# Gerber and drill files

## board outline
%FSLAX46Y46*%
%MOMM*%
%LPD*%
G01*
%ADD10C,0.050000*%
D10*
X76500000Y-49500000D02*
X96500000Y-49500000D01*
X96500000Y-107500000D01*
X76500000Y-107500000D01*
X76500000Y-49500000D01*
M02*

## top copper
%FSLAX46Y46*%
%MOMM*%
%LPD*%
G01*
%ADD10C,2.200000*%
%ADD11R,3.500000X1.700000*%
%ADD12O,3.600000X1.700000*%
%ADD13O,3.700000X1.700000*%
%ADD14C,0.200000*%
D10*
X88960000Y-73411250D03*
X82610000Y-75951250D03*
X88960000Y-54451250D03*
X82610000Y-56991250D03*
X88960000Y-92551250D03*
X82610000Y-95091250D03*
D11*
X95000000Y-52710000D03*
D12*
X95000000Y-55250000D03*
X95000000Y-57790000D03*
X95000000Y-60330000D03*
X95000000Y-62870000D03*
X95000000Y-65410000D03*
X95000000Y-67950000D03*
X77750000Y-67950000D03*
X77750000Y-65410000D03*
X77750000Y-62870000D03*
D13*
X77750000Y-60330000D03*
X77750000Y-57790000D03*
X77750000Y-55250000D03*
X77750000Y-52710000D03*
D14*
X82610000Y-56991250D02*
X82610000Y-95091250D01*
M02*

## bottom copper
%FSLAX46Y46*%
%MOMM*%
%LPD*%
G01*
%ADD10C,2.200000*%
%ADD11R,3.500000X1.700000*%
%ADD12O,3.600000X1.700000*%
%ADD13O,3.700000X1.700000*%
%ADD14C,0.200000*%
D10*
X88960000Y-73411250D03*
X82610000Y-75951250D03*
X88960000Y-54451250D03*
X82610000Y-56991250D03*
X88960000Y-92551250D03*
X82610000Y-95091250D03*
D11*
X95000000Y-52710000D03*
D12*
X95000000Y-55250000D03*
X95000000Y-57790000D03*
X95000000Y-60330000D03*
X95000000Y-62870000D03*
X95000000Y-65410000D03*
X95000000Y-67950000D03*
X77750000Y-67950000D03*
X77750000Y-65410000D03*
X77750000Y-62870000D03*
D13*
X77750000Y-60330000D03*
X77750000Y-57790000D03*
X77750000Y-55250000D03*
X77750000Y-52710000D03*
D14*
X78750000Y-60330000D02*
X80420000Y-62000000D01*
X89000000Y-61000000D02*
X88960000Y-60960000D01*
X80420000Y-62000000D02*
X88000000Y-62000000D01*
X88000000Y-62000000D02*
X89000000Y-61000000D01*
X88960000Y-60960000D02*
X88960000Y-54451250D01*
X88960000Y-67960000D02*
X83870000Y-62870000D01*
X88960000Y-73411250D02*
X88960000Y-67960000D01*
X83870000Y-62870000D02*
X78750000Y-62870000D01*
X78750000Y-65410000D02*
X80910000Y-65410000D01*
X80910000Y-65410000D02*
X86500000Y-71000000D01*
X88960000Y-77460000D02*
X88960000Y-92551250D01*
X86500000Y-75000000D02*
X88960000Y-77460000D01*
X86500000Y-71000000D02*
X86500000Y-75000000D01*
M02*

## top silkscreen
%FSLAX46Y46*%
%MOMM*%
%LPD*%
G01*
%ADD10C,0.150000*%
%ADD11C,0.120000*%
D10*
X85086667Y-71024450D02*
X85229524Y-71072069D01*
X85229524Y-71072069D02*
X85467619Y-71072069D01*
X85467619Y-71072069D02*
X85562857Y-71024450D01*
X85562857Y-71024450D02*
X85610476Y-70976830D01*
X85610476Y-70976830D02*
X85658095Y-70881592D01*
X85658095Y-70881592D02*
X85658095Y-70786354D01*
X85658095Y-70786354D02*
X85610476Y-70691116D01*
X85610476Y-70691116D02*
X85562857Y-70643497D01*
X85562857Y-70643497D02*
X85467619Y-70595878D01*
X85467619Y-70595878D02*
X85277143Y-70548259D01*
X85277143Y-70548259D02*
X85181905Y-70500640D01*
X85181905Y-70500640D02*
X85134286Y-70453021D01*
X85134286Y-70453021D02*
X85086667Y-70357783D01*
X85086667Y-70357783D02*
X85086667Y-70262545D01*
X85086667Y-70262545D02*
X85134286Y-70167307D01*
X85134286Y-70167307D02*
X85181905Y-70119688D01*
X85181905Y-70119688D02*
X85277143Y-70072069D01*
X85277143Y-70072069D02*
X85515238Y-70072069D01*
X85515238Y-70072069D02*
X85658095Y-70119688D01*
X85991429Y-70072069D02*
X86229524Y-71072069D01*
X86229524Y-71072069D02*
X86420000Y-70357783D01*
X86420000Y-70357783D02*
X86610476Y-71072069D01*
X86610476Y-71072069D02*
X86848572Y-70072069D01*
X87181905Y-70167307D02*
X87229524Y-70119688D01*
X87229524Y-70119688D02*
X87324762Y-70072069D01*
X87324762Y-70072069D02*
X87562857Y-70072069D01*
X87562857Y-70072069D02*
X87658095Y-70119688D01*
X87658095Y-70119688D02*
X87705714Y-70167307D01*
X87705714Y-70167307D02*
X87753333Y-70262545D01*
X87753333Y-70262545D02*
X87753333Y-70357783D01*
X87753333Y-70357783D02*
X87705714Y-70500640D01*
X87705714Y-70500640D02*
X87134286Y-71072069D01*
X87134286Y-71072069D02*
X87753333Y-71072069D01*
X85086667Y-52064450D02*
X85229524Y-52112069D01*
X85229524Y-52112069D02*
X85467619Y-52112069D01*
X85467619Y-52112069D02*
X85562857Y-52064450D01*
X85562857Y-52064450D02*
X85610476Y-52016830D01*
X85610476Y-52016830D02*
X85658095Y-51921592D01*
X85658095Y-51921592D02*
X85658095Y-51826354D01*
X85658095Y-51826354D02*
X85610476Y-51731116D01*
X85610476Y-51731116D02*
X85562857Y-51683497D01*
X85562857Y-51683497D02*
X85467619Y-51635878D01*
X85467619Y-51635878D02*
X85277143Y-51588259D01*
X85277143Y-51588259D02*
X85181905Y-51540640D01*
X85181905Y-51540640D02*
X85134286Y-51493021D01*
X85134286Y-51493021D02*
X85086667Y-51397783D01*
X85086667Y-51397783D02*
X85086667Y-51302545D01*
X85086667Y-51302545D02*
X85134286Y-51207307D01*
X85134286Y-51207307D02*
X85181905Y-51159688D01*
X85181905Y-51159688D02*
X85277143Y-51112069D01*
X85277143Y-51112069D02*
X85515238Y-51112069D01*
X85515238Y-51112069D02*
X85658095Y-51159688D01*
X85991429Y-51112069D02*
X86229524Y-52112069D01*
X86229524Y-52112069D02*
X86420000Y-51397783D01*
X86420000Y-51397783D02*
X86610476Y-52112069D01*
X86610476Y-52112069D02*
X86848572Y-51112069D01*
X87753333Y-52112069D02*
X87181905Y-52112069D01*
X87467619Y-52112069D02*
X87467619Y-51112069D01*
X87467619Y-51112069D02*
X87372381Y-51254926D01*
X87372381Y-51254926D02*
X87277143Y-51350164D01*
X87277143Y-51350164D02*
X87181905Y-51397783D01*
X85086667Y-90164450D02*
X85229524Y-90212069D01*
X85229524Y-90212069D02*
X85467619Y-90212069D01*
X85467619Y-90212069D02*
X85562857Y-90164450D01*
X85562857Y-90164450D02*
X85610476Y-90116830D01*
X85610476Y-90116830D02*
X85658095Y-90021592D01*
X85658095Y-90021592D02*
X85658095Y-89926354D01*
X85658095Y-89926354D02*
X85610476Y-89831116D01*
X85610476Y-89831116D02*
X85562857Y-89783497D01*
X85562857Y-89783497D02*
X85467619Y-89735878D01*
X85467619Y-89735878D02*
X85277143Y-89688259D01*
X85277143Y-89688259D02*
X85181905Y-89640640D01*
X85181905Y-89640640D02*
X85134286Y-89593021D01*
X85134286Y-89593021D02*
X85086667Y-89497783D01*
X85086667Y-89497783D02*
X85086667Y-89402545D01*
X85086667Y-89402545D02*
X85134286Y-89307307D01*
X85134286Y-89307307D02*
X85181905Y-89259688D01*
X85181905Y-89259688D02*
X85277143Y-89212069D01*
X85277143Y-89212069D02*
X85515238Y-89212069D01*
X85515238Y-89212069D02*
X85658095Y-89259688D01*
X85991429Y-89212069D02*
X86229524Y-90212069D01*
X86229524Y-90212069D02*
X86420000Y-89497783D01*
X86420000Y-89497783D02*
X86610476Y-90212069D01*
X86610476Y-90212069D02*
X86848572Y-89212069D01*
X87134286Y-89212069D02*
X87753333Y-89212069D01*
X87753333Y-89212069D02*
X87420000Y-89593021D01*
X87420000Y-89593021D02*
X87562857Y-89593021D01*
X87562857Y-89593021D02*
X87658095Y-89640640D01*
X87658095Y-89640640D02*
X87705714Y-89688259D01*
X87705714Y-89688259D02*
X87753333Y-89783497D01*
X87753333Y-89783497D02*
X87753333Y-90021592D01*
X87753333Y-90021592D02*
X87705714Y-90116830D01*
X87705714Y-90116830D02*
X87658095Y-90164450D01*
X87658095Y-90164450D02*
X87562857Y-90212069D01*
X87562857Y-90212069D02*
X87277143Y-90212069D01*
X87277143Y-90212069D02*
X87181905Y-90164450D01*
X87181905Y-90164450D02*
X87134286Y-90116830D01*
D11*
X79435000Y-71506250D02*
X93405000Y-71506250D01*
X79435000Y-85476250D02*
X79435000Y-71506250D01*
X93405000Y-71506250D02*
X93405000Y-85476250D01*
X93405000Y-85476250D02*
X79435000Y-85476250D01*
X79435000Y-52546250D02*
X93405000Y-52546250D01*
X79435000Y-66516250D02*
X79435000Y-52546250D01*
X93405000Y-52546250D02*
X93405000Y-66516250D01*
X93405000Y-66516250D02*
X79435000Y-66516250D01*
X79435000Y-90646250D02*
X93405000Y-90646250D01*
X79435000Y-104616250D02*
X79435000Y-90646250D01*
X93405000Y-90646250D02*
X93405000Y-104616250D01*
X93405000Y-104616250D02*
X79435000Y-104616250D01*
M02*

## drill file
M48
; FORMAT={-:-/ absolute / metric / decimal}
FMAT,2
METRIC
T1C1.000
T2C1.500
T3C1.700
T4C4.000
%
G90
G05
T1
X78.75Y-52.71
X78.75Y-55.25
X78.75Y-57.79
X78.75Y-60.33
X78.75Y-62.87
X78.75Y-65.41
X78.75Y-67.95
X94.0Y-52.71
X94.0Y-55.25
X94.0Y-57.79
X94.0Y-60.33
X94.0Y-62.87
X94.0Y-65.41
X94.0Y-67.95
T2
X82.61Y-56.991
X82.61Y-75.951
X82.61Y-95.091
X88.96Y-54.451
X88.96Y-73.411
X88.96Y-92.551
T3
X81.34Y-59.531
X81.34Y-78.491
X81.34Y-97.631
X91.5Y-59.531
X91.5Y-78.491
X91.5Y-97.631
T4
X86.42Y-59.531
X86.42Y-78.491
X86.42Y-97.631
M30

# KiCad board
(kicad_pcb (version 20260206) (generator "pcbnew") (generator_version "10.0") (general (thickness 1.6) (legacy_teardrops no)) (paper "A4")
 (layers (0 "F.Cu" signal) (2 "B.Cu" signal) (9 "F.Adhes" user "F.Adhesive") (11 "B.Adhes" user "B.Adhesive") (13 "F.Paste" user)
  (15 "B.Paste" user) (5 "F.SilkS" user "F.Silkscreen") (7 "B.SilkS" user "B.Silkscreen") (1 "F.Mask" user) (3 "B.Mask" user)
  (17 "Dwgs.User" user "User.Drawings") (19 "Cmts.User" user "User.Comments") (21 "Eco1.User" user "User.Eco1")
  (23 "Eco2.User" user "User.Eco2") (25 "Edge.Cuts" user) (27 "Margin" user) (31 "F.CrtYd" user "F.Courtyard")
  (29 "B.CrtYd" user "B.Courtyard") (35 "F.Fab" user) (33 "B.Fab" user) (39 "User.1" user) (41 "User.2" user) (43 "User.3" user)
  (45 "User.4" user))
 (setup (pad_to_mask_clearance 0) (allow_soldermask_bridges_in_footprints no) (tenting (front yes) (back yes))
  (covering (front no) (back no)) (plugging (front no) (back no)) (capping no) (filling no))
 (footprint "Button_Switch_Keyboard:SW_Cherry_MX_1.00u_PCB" (layer "F.Cu") (at 88.96 73.41125)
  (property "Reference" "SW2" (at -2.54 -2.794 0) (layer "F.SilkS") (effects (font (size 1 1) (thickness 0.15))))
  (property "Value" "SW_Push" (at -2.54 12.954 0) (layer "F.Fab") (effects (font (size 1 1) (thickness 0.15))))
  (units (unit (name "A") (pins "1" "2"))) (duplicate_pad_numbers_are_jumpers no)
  (fp_line (start -9.525 -1.905) (end 4.445 -1.905) (stroke (width 0.12) (type solid)) (layer "F.SilkS"))
  (fp_line (start -9.525 12.065) (end -9.525 -1.905) (stroke (width 0.12) (type solid)) (layer "F.SilkS"))
  (fp_line (start 4.445 -1.905) (end 4.445 12.065) (stroke (width 0.12) (type solid)) (layer "F.SilkS"))
  (fp_line (start 4.445 12.065) (end -9.525 12.065) (stroke (width 0.12) (type solid)) (layer "F.SilkS"))
  (pad "" np_thru_hole circle (at -7.62 5.08) (size 1.7 1.7) (drill 1.7) (layers "*.Cu" "*.Mask"))
  (pad "" np_thru_hole circle (at -2.54 5.08) (size 4 4) (drill 4) (layers "*.Cu" "*.Mask"))
  (pad "" np_thru_hole circle (at 2.54 5.08) (size 1.7 1.7) (drill 1.7) (layers "*.Cu" "*.Mask"))
  (pad "1" thru_hole circle (at 0 0) (size 2.2 2.2) (drill 1.5) (layers "*.Cu" "*.Mask") (remove_unused_layers no)
   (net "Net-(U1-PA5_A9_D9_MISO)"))
  (pad "2" thru_hole circle (at -6.35 2.54) (size 2.2 2.2) (drill 1.5) (layers "*.Cu" "*.Mask") (remove_unused_layers no) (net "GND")))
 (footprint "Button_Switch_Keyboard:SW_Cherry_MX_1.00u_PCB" (layer "F.Cu") (at 88.96 54.45125)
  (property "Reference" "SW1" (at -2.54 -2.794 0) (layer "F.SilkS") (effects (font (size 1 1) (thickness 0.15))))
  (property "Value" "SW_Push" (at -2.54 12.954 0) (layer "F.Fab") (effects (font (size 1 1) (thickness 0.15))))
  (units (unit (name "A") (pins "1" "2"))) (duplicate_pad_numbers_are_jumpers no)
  (fp_line (start -9.525 -1.905) (end 4.445 -1.905) (stroke (width 0.12) (type solid)) (layer "F.SilkS"))
  (fp_line (start -9.525 12.065) (end -9.525 -1.905) (stroke (width 0.12) (type solid)) (layer "F.SilkS"))
  (fp_line (start 4.445 -1.905) (end 4.445 12.065) (stroke (width 0.12) (type solid)) (layer "F.SilkS"))
  (fp_line (start 4.445 12.065) (end -9.525 12.065) (stroke (width 0.12) (type solid)) (layer "F.SilkS"))
  (pad "" np_thru_hole circle (at -7.62 5.08) (size 1.7 1.7) (drill 1.7) (layers "*.Cu" "*.Mask"))
  (pad "" np_thru_hole circle (at -2.54 5.08) (size 4 4) (drill 4) (layers "*.Cu" "*.Mask"))
  (pad "" np_thru_hole circle (at 2.54 5.08) (size 1.7 1.7) (drill 1.7) (layers "*.Cu" "*.Mask"))
  (pad "1" thru_hole circle (at 0 0) (size 2.2 2.2) (drill 1.5) (layers "*.Cu" "*.Mask") (remove_unused_layers no)
   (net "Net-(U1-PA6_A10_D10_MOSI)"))
  (pad "2" thru_hole circle (at -6.35 2.54) (size 2.2 2.2) (drill 1.5) (layers "*.Cu" "*.Mask") (remove_unused_layers no) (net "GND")))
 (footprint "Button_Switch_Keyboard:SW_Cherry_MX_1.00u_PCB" (layer "F.Cu") (at 88.96 92.55125)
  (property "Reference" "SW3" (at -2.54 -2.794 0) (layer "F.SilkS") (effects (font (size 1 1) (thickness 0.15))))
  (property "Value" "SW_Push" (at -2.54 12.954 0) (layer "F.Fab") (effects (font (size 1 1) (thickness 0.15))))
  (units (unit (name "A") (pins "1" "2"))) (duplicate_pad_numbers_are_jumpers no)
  (fp_line (start -9.525 -1.905) (end 4.445 -1.905) (stroke (width 0.12) (type solid)) (layer "F.SilkS"))
  (fp_line (start -9.525 12.065) (end -9.525 -1.905) (stroke (width 0.12) (type solid)) (layer "F.SilkS"))
  (fp_line (start 4.445 -1.905) (end 4.445 12.065) (stroke (width 0.12) (type solid)) (layer "F.SilkS"))
  (fp_line (start 4.445 12.065) (end -9.525 12.065) (stroke (width 0.12) (type solid)) (layer "F.SilkS"))
  (pad "" np_thru_hole circle (at -7.62 5.08) (size 1.7 1.7) (drill 1.7) (layers "*.Cu" "*.Mask"))
  (pad "" np_thru_hole circle (at -2.54 5.08) (size 4 4) (drill 4) (layers "*.Cu" "*.Mask"))
  (pad "" np_thru_hole circle (at 2.54 5.08) (size 1.7 1.7) (drill 1.7) (layers "*.Cu" "*.Mask"))
  (pad "1" thru_hole circle (at 0 0) (size 2.2 2.2) (drill 1.5) (layers "*.Cu" "*.Mask") (remove_unused_layers no)
   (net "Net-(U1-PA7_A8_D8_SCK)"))
  (pad "2" thru_hole circle (at -6.35 2.54) (size 2.2 2.2) (drill 1.5) (layers "*.Cu" "*.Mask") (remove_unused_layers no) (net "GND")))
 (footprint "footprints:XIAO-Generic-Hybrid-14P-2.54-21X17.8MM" (layer "B.Cu") (at 86.375 60.33 180)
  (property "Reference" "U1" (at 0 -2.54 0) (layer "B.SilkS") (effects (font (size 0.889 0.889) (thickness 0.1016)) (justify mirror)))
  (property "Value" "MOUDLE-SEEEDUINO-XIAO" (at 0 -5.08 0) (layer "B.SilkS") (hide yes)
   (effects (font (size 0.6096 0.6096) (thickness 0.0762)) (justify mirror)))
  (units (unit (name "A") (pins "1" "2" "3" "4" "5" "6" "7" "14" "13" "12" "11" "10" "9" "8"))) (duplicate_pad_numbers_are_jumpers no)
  (pad "1" thru_hole rect (at -7.625 7.62 180) (size 3.5 1.7) (drill 1 (offset -1 0)) (layers "*.Cu" "*.Mask") (remove_unused_layers no)
   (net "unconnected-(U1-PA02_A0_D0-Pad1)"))
  (pad "2" thru_hole oval (at -7.625 5.08 180) (size 3.6 1.7) (drill 1 (offset -1 0)) (layers "*.Cu" "*.Mask") (remove_unused_layers no)
   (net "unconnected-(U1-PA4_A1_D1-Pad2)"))
  (pad "3" thru_hole oval (at -7.625 2.54 180) (size 3.6 1.7) (drill 1 (offset -1 0)) (layers "*.Cu" "*.Mask") (remove_unused_layers no)
   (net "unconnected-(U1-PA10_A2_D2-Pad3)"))
  (pad "4" thru_hole oval (at -7.625 0 180) (size 3.6 1.7) (drill 1 (offset -1 0)) (layers "*.Cu" "*.Mask") (remove_unused_layers no)
   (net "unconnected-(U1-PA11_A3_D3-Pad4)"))
  (pad "5" thru_hole oval (at -7.625 -2.54 180) (size 3.6 1.7) (drill 1 (offset -1 0)) (layers "*.Cu" "*.Mask") (remove_unused_layers no)
   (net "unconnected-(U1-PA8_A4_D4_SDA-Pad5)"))
  (pad "6" thru_hole oval (at -7.625 -5.08) (size 3.6 1.7) (drill 1 (offset 1 0)) (layers "*.Cu" "*.Mask") (remove_unused_layers no)
   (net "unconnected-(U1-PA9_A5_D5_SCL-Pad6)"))
  (pad "7" thru_hole oval (at -7.625 -7.62 180) (size 3.6 1.7) (drill 1 (offset -1 0)) (layers "*.Cu" "*.Mask") (remove_unused_layers no)
   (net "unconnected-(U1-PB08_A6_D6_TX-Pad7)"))
  (pad "8" thru_hole oval (at 7.625 -7.62 180) (size 3.6 1.7) (drill 1 (offset 1 0)) (layers "*.Cu" "*.Mask") (remove_unused_layers no)
   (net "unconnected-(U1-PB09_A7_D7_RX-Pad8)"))
  (pad "9" thru_hole oval (at 7.625 -5.08 180) (size 3.6 1.7) (drill 1 (offset 1 0)) (layers "*.Cu" "*.Mask") (remove_unused_layers no)
   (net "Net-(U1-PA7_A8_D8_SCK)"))
  (pad "10" thru_hole oval (at 7.625 -2.54 180) (size 3.6 1.7) (drill 1 (offset 1 0)) (layers "*.Cu" "*.Mask") (remove_unused_layers no)
   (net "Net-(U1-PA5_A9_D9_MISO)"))
  (pad "11" thru_hole oval (at 7.625 0 180) (size 3.7 1.7) (drill 1 (offset 1 0)) (layers "*.Cu" "*.Mask") (remove_unused_layers no)
   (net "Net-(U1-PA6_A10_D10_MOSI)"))
  (pad "12" thru_hole oval (at 7.625 2.54 180) (size 3.7 1.7) (drill 1 (offset 1 0)) (layers "*.Cu" "*.Mask") (remove_unused_layers no)
   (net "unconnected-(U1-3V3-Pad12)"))
  (pad "13" thru_hole oval (at 7.625 5.08 180) (size 3.7 1.7) (drill 1 (offset 1 0)) (layers "*.Cu" "*.Mask") (remove_unused_layers no)
   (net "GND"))
  (pad "14" thru_hole oval (at 7.625 7.62 180) (size 3.7 1.7) (drill 1 (offset 1 0)) (layers "*.Cu" "*.Mask") (remove_unused_layers no)
   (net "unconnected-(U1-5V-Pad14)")))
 (gr_rect (start 76.5 49.5) (end 96.5 107.5) (stroke (width 0.05) (type default)) (fill no) (layer "Edge.Cuts"))
 (segment (start 78.75 60.33) (end 80.42 62) (width 0.2) (layer "B.Cu") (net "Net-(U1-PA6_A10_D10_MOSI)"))
 (segment (start 89 61) (end 88.96 60.96) (width 0.2) (layer "B.Cu") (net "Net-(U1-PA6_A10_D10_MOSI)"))
 (segment (start 80.42 62) (end 88 62) (width 0.2) (layer "B.Cu") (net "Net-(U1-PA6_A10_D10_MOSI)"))
 (segment (start 88 62) (end 89 61) (width 0.2) (layer "B.Cu") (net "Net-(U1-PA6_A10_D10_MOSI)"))
 (segment (start 88.96 60.96) (end 88.96 54.45125) (width 0.2) (layer "B.Cu") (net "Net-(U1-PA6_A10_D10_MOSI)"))
 (segment (start 82.61 56.99125) (end 82.61 95.09125) (width 0.2) (layer "F.Cu") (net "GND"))
 (segment (start 88.96 67.96) (end 83.87 62.87) (width 0.2) (layer "B.Cu") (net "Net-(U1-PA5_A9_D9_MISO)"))
 (segment (start 88.96 73.41125) (end 88.96 67.96) (width 0.2) (layer "B.Cu") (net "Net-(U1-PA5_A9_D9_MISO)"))
 (segment (start 83.87 62.87) (end 78.75 62.87) (width 0.2) (layer "B.Cu") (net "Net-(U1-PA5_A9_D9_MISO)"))
 (segment (start 78.75 65.41) (end 80.91 65.41) (width 0.2) (layer "B.Cu") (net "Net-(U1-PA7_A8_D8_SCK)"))
 (segment (start 80.91 65.41) (end 86.5 71) (width 0.2) (layer "B.Cu") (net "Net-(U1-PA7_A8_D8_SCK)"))
 (segment (start 88.96 77.46) (end 88.96 92.55125) (width 0.2) (layer "B.Cu") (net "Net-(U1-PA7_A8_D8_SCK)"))
 (segment (start 86.5 75) (end 88.96 77.46) (width 0.2) (layer "B.Cu") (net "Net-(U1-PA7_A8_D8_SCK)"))
 (segment (start 86.5 71) (end 86.5 75) (width 0.2) (layer "B.Cu") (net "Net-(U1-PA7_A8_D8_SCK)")))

